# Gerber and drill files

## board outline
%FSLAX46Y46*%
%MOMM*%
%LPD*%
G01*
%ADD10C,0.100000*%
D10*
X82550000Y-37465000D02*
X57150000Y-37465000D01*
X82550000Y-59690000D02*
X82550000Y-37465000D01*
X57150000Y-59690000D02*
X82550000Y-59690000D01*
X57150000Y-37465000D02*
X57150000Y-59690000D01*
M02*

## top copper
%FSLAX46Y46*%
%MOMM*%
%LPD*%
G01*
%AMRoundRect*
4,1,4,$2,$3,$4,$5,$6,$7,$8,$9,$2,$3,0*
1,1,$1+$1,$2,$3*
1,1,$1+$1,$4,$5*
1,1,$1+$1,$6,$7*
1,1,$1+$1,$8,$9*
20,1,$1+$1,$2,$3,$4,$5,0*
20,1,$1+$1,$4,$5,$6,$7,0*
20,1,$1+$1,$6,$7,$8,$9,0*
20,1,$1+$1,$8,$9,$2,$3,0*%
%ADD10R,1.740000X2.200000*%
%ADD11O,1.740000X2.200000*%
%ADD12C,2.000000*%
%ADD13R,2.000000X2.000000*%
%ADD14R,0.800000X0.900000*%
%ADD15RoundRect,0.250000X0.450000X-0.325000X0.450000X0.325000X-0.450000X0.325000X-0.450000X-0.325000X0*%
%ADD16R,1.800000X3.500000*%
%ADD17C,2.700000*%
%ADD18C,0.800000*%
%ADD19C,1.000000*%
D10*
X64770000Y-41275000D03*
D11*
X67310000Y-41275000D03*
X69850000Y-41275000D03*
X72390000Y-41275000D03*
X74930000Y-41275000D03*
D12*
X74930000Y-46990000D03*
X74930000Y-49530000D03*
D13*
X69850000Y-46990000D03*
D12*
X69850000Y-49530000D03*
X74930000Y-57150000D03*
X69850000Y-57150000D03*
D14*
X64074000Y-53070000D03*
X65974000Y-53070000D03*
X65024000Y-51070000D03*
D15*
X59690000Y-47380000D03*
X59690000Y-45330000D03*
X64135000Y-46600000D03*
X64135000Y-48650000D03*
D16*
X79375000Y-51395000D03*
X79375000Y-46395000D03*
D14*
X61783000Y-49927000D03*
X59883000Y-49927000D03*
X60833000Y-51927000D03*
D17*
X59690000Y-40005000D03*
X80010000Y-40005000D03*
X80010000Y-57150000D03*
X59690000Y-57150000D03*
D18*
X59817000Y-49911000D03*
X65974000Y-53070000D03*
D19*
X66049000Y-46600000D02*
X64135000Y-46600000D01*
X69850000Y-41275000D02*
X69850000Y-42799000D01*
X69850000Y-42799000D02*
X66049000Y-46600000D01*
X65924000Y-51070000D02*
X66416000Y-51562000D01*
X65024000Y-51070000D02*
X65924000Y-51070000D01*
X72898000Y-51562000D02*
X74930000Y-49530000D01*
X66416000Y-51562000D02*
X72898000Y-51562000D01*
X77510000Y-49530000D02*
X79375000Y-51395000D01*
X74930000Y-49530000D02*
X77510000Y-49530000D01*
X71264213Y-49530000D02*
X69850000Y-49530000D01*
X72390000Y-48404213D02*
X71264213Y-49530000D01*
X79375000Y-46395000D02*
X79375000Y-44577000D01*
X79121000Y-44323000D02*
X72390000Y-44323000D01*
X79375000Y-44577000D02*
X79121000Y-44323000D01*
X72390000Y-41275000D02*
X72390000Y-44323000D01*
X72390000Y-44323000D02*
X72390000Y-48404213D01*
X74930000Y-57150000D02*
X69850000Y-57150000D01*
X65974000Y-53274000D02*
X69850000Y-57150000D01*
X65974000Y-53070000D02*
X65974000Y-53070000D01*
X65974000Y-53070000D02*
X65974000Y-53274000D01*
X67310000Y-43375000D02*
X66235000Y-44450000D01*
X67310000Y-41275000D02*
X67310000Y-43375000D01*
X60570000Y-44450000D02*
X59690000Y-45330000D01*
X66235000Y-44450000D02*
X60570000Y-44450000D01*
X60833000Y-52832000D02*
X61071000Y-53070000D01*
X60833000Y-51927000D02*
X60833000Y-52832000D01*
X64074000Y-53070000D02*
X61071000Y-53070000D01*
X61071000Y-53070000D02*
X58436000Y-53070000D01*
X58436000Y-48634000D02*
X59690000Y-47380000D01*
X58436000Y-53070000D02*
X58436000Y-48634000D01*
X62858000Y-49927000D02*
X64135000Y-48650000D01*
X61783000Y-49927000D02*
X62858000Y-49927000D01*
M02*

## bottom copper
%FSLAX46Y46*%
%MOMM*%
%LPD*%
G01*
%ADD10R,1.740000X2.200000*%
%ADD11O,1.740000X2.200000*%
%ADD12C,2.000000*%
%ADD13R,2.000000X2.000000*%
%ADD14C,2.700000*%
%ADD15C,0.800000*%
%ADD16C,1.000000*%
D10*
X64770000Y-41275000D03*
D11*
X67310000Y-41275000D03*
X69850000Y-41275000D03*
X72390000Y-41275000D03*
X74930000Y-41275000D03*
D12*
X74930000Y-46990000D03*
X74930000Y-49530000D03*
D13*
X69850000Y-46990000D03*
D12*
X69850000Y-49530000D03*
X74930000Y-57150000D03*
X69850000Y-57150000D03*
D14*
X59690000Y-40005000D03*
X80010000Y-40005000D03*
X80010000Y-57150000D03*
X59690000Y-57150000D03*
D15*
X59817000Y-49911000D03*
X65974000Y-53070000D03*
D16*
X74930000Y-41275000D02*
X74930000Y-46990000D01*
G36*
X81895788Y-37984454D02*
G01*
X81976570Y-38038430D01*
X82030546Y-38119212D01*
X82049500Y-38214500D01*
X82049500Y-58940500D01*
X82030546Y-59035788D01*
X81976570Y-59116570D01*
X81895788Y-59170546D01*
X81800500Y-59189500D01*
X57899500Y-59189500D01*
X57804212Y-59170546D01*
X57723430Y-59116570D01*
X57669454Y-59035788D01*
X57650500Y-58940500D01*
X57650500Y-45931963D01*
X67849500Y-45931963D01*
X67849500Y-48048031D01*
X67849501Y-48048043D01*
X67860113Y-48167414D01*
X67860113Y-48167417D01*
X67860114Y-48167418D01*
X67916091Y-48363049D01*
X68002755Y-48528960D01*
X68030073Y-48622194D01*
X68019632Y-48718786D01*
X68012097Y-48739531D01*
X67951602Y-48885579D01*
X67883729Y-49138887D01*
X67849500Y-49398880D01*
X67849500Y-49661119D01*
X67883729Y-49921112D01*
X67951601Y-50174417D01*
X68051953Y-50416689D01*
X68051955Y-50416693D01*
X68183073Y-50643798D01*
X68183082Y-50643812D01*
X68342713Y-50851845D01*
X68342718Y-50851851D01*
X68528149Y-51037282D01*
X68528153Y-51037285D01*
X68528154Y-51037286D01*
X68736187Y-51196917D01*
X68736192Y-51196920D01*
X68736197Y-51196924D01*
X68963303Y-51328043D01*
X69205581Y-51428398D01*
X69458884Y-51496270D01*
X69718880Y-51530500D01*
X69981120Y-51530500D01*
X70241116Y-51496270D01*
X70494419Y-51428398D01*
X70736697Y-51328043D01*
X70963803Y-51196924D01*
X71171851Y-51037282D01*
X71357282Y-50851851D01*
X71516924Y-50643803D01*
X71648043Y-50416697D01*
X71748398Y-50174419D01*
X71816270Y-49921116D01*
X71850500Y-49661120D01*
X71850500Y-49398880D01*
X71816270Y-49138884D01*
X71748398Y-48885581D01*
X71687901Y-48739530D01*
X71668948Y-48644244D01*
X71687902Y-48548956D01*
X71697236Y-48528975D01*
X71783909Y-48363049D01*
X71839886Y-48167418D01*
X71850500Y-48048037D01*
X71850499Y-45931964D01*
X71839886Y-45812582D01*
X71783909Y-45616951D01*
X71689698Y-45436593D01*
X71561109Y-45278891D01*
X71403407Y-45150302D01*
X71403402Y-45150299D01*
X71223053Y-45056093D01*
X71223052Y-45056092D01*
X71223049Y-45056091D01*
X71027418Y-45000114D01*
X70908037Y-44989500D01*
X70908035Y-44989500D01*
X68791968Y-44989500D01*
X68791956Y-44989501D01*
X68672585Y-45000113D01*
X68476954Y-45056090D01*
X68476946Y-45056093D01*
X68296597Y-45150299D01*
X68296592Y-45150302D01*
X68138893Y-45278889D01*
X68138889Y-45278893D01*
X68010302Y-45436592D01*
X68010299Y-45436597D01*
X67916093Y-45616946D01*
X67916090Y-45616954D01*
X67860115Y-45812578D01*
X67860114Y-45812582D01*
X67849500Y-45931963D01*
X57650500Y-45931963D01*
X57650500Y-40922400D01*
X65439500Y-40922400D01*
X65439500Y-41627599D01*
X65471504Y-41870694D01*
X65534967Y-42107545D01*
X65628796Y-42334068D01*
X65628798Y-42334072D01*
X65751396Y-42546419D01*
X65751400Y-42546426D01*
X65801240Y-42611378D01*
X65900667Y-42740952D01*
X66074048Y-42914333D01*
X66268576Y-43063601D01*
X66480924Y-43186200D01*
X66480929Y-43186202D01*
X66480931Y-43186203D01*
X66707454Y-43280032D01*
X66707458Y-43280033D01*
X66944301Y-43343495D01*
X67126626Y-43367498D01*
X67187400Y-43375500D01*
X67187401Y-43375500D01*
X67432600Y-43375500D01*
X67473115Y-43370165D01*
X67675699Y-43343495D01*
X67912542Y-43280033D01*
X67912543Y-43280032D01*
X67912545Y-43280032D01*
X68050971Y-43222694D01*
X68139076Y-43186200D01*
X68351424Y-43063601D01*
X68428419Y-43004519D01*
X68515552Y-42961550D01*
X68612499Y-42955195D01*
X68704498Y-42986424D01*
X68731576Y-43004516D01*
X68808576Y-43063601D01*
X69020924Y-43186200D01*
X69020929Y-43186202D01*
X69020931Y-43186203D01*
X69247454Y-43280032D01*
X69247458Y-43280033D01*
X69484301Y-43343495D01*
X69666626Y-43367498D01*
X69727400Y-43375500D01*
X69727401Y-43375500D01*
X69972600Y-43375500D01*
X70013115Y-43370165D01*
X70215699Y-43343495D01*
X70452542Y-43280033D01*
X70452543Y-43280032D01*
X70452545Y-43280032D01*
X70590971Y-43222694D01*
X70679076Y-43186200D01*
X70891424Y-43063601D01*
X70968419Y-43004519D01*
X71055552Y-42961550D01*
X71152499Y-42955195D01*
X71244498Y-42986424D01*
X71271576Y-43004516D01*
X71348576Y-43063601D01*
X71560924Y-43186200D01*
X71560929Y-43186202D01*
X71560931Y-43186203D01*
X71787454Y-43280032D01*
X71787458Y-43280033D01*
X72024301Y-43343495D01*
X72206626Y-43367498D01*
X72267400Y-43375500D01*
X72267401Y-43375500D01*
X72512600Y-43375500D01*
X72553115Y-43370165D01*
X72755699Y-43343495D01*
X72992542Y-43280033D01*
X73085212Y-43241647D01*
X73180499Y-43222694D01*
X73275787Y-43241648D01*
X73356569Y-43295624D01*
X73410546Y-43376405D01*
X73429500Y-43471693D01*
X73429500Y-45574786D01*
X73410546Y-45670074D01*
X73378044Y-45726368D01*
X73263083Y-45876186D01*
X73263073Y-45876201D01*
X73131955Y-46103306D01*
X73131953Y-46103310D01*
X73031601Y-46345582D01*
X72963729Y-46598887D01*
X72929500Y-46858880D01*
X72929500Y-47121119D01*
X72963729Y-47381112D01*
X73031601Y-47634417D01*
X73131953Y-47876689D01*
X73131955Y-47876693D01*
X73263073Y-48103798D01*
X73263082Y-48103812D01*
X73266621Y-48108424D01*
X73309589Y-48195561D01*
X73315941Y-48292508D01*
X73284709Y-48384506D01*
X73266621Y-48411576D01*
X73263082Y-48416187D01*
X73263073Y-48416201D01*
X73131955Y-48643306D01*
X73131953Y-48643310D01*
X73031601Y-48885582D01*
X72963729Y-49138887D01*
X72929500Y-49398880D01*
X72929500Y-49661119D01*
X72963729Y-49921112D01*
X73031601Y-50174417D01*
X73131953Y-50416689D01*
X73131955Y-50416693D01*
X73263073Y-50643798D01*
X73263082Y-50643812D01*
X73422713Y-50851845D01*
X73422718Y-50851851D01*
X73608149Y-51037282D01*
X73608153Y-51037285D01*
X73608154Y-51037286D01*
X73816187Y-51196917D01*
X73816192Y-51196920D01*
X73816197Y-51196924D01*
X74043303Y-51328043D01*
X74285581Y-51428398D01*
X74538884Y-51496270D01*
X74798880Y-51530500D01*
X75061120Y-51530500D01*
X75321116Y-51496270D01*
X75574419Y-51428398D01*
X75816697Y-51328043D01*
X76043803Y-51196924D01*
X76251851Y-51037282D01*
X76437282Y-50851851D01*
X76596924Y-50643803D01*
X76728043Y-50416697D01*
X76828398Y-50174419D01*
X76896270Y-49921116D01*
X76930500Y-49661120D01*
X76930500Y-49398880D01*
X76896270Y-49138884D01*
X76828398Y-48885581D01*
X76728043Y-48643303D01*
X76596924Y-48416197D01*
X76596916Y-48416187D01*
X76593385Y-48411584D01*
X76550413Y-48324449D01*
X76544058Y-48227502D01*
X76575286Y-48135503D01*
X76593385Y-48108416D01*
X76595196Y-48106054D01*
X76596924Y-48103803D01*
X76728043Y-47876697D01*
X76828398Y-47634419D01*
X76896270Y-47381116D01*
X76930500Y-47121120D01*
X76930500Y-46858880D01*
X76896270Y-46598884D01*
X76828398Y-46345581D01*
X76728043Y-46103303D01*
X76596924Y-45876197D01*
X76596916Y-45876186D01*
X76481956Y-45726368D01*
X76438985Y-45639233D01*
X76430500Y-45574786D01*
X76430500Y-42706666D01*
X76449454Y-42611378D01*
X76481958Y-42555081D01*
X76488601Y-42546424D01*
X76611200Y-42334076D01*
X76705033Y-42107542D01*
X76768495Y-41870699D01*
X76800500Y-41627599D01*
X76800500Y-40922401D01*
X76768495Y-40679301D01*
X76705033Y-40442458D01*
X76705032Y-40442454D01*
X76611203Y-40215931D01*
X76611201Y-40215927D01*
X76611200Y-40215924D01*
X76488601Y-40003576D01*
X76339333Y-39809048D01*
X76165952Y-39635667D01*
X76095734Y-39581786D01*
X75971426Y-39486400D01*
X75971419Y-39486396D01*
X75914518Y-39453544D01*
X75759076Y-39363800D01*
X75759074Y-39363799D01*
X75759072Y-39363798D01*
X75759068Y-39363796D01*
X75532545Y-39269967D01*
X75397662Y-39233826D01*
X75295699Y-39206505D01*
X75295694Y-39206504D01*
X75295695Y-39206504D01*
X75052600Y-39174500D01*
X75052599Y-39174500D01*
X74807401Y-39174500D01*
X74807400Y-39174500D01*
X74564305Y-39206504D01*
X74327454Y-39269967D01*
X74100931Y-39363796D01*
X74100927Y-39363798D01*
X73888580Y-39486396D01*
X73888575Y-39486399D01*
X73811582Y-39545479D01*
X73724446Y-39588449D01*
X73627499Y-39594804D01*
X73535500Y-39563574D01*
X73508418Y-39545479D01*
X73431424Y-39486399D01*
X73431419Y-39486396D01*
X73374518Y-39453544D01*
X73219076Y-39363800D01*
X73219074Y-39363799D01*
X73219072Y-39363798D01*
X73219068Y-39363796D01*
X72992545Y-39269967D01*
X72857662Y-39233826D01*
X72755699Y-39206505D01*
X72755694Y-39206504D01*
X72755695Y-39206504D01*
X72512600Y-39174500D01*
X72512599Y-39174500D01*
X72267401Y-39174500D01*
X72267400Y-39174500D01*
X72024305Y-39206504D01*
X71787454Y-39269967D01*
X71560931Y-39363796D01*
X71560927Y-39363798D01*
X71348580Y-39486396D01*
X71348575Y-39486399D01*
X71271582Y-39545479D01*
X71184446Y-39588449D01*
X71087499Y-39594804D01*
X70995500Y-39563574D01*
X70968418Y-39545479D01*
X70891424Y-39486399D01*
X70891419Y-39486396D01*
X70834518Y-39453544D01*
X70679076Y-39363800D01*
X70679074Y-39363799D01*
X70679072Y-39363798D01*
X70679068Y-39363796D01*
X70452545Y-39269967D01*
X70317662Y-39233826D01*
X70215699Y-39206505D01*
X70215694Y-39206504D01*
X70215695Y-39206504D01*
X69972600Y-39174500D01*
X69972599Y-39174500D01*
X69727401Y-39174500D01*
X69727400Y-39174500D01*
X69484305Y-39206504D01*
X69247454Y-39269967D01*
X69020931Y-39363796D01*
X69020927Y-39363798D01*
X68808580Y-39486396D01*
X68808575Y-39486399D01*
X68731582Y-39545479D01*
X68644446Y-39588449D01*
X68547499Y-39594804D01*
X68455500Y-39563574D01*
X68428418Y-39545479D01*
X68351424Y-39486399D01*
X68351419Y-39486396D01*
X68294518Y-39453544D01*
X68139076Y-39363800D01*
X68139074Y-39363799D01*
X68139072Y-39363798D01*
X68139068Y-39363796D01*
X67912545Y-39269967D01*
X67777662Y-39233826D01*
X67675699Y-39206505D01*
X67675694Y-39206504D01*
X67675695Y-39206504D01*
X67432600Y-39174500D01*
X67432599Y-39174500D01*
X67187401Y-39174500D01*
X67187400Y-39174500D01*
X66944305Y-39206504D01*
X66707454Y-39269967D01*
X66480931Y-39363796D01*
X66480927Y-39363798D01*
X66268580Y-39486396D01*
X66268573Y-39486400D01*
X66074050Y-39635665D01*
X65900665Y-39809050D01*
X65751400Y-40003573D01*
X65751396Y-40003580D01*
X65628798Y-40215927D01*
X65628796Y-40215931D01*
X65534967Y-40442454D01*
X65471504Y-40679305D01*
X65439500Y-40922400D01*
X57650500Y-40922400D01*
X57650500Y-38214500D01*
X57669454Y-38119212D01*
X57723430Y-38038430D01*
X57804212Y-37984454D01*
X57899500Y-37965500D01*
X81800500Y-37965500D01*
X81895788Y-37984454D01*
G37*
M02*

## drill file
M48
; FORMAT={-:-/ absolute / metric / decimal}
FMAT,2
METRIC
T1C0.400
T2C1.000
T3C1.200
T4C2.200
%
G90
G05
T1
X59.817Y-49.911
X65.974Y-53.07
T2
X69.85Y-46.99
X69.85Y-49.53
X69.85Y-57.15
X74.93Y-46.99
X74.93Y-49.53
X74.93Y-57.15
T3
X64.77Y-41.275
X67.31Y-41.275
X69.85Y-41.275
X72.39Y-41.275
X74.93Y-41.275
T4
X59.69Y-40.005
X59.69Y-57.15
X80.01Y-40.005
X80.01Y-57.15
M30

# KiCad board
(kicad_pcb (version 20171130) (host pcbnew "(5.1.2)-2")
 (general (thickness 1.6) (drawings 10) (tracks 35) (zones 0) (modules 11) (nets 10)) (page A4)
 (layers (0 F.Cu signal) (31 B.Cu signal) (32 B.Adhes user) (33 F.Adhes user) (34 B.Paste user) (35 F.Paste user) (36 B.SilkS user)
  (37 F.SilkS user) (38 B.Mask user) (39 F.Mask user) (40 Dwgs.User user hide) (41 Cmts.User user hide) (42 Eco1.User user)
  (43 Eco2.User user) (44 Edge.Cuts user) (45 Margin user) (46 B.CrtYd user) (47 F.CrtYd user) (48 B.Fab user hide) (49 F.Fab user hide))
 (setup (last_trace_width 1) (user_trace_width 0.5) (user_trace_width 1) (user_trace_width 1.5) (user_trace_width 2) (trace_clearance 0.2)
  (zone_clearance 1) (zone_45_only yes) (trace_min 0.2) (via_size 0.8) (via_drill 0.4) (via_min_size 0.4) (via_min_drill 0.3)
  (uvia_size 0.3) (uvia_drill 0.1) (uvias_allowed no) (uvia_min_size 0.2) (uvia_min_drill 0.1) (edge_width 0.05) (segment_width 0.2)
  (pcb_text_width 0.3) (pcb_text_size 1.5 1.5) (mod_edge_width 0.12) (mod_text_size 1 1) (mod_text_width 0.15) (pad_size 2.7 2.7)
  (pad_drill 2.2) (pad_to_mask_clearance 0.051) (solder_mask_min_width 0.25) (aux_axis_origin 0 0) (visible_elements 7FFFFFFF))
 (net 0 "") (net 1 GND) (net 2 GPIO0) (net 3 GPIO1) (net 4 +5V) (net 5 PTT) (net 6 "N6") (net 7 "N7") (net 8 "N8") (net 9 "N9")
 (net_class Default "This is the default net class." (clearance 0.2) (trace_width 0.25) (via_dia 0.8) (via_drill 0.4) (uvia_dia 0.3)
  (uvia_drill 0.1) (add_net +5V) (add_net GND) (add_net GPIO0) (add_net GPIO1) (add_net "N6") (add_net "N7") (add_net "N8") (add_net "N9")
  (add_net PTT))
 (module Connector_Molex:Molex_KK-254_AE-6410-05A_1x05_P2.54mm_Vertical (layer F.Cu) (at 64.77 41.275)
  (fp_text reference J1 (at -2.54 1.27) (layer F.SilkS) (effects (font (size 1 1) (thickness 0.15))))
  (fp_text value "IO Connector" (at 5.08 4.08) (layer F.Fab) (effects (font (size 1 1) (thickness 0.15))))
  (pad 1 thru_hole rect (at 0 0) (size 1.74 2.2) (drill 1.2) (layers *.Cu *.Mask) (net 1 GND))
  (pad 2 thru_hole oval (at 2.54 0) (size 1.74 2.2) (drill 1.2) (layers *.Cu *.Mask) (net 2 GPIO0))
  (pad 3 thru_hole oval (at 5.08 0) (size 1.74 2.2) (drill 1.2) (layers *.Cu *.Mask) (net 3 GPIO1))
  (pad 4 thru_hole oval (at 7.62 0) (size 1.74 2.2) (drill 1.2) (layers *.Cu *.Mask) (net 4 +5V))
  (pad 5 thru_hole oval (at 10.16 0) (size 1.74 2.2) (drill 1.2) (layers *.Cu *.Mask) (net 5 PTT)))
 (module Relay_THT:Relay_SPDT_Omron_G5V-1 (layer F.Cu) (at 69.85 46.99)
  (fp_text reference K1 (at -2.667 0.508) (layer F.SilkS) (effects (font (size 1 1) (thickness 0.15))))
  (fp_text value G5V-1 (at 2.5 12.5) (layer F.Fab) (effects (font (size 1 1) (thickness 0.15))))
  (pad 10 thru_hole circle (at 5.08 0) (size 2 2) (drill 1) (layers *.Cu *.Mask) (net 5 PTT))
  (pad 9 thru_hole circle (at 5.08 2.54) (size 2 2) (drill 1) (layers *.Cu *.Mask) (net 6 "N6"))
  (pad 1 thru_hole rect (at 0 0) (size 2 2) (drill 1) (layers *.Cu *.Mask) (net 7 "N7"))
  (pad 2 thru_hole circle (at 0 2.54) (size 2 2) (drill 1) (layers *.Cu *.Mask) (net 4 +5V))
  (pad 6 thru_hole circle (at 5.08 10.16) (size 2 2) (drill 1) (layers *.Cu *.Mask) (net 1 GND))
  (pad 5 thru_hole circle (at 0 10.16) (size 2 2) (drill 1) (layers *.Cu *.Mask) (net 1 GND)))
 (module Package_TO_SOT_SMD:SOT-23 (layer F.Cu) (at 65.024 52.07 90)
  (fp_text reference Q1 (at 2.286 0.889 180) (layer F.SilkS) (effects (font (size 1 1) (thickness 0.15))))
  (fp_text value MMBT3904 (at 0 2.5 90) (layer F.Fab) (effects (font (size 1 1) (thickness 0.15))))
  (pad 1 smd rect (at -1 -0.95 90) (size 0.9 0.8) (layers F.Cu F.Paste F.Mask) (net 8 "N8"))
  (pad 2 smd rect (at -1 0.95 90) (size 0.9 0.8) (layers F.Cu F.Paste F.Mask) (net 1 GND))
  (pad 3 smd rect (at 1 0 90) (size 0.9 0.8) (layers F.Cu F.Paste F.Mask) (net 6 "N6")))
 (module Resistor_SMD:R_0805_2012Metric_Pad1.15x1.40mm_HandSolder (layer F.Cu) (at 59.69 46.355 90)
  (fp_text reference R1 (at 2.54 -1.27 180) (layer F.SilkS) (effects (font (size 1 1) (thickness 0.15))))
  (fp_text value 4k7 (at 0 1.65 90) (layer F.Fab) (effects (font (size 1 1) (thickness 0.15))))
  (pad 1 smd roundrect (at -1.025 0 90) (size 1.15 1.4) (layers F.Cu F.Paste F.Mask) (roundrect_rratio 0.217391) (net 8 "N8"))
  (pad 2 smd roundrect (at 1.025 0 90) (size 1.15 1.4) (layers F.Cu F.Paste F.Mask) (roundrect_rratio 0.217391) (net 2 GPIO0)))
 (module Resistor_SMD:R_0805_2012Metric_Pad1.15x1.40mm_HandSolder (layer F.Cu) (at 64.135 47.625 90)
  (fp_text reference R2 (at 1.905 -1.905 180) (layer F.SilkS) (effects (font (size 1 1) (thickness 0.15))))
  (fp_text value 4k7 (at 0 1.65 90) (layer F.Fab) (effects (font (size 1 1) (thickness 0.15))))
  (pad 2 smd roundrect (at 1.025 0 90) (size 1.15 1.4) (layers F.Cu F.Paste F.Mask) (roundrect_rratio 0.217391) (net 3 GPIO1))
  (pad 1 smd roundrect (at -1.025 0 90) (size 1.15 1.4) (layers F.Cu F.Paste F.Mask) (roundrect_rratio 0.217391) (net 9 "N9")))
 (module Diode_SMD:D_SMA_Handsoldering (layer F.Cu) (at 79.375 48.895 90)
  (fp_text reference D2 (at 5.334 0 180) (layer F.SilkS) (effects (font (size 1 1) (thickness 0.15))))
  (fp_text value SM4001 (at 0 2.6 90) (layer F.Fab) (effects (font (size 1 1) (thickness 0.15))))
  (pad 1 smd rect (at -2.5 0 90) (size 3.5 1.8) (layers F.Cu F.Paste F.Mask) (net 6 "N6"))
  (pad 2 smd rect (at 2.5 0 90) (size 3.5 1.8) (layers F.Cu F.Paste F.Mask) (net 4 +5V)))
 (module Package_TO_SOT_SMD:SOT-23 (layer F.Cu) (at 60.833 50.927 270)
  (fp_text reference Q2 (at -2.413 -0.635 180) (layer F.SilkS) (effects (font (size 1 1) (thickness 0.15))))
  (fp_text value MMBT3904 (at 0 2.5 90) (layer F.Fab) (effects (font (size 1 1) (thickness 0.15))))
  (pad 1 smd rect (at -1 -0.95 270) (size 0.9 0.8) (layers F.Cu F.Paste F.Mask) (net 9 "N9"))
  (pad 2 smd rect (at -1 0.95 270) (size 0.9 0.8) (layers F.Cu F.Paste F.Mask) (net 1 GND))
  (pad 3 smd rect (at 1 0 270) (size 0.9 0.8) (layers F.Cu F.Paste F.Mask) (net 8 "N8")))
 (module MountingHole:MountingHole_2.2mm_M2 (layer F.Cu) (at 59.69 40.005)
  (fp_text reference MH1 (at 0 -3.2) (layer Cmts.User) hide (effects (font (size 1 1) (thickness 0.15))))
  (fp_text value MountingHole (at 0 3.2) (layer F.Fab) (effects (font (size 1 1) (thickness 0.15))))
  (pad "" thru_hole circle (at 0 0) (size 2.7 2.7) (drill 2.2) (layers *.Cu *.Mask) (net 1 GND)))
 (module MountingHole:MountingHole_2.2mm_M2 (layer F.Cu) (at 80.01 40.005)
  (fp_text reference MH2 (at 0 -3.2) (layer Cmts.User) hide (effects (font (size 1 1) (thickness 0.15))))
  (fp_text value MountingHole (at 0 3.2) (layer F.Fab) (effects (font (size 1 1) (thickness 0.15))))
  (pad 1 thru_hole circle (at 0 0) (size 2.7 2.7) (drill 2.2) (layers *.Cu *.Mask) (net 1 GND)))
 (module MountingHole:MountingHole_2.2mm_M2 (layer F.Cu) (at 80.01 57.15)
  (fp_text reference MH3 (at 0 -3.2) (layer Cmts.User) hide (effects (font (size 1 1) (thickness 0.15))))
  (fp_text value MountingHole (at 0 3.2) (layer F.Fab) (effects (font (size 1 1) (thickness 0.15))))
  (pad "" thru_hole circle (at 0 0) (size 2.7 2.7) (drill 2.2) (layers *.Cu *.Mask) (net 1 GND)))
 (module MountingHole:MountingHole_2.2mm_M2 (layer F.Cu) (at 59.69 57.15)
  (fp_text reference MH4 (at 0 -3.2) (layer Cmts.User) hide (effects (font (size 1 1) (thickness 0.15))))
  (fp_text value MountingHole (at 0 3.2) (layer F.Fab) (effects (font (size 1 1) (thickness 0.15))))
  (pad "" thru_hole circle (at 0 0) (size 2.7 2.7) (drill 2.2) (layers *.Cu *.Mask) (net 1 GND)))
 (gr_line (start 82.55 37.465) (end 57.15 37.465) (layer Edge.Cuts) (width 0.1))
 (gr_line (start 82.55 59.69) (end 82.55 37.465) (layer Edge.Cuts) (width 0.1))
 (gr_line (start 57.15 59.69) (end 82.55 59.69) (layer Edge.Cuts) (width 0.1))
 (gr_line (start 57.15 37.465) (end 57.15 59.69) (layer Edge.Cuts) (width 0.1))
 (via (at 59.817 49.911) (size 0.8) (drill 0.4) (layers F.Cu B.Cu) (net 1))
 (segment (start 66.049 46.6) (end 64.135 46.6) (width 1) (layer F.Cu) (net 3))
 (segment (start 69.85 41.275) (end 69.85 42.799) (width 1) (layer F.Cu) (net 3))
 (segment (start 69.85 42.799) (end 66.049 46.6) (width 1) (layer F.Cu) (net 3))
 (segment (start 65.924 51.07) (end 66.416 51.562) (width 1) (layer F.Cu) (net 6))
 (segment (start 65.024 51.07) (end 65.924 51.07) (width 1) (layer F.Cu) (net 6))
 (segment (start 72.898 51.562) (end 74.93 49.53) (width 1) (layer F.Cu) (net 6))
 (segment (start 66.416 51.562) (end 72.898 51.562) (width 1) (layer F.Cu) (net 6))
 (segment (start 77.51 49.53) (end 79.375 51.395) (width 1) (layer F.Cu) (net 6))
 (segment (start 74.93 49.53) (end 77.51 49.53) (width 1) (layer F.Cu) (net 6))
 (segment (start 71.264213 49.53) (end 69.85 49.53) (width 1) (layer F.Cu) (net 4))
 (segment (start 72.39 48.404213) (end 71.264213 49.53) (width 1) (layer F.Cu) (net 4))
 (segment (start 79.375 46.395) (end 79.375 44.577) (width 1) (layer F.Cu) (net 4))
 (segment (start 79.121 44.323) (end 72.39 44.323) (width 1) (layer F.Cu) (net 4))
 (segment (start 79.375 44.577) (end 79.121 44.323) (width 1) (layer F.Cu) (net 4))
 (segment (start 72.39 41.275) (end 72.39 44.323) (width 1) (layer F.Cu) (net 4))
 (segment (start 72.39 44.323) (end 72.39 48.404213) (width 1) (layer F.Cu) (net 4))
 (segment (start 74.93 57.15) (end 69.85 57.15) (width 1) (layer F.Cu) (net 1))
 (segment (start 65.974 53.274) (end 69.85 57.15) (width 1) (layer F.Cu) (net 1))
 (segment (start 65.974 53.07) (end 65.974 53.07) (width 1) (layer F.Cu) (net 1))
 (segment (start 65.974 53.07) (end 65.974 53.274) (width 1) (layer F.Cu) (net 1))
 (via (at 65.974 53.07) (size 0.8) (drill 0.4) (layers F.Cu B.Cu) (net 1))
 (segment (start 67.31 43.375) (end 66.235 44.45) (width 1) (layer F.Cu) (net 2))
 (segment (start 67.31 41.275) (end 67.31 43.375) (width 1) (layer F.Cu) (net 2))
 (segment (start 60.57 44.45) (end 59.69 45.33) (width 1) (layer F.Cu) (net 2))
 (segment (start 66.235 44.45) (end 60.57 44.45) (width 1) (layer F.Cu) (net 2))
 (segment (start 74.93 41.275) (end 74.93 46.99) (width 1) (layer B.Cu) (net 5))
 (segment (start 60.833 52.832) (end 61.071 53.07) (width 1) (layer F.Cu) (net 8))
 (segment (start 60.833 51.927) (end 60.833 52.832) (width 1) (layer F.Cu) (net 8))
 (segment (start 64.074 53.07) (end 61.071 53.07) (width 1) (layer F.Cu) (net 8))
 (segment (start 61.071 53.07) (end 58.436 53.07) (width 1) (layer F.Cu) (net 8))
 (segment (start 58.436 48.634) (end 59.69 47.38) (width 1) (layer F.Cu) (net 8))
 (segment (start 58.436 53.07) (end 58.436 48.634) (width 1) (layer F.Cu) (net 8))
 (segment (start 62.858 49.927) (end 64.135 48.65) (width 1) (layer F.Cu) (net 9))
 (segment (start 61.783 49.927) (end 62.858 49.927) (width 1) (layer F.Cu) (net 9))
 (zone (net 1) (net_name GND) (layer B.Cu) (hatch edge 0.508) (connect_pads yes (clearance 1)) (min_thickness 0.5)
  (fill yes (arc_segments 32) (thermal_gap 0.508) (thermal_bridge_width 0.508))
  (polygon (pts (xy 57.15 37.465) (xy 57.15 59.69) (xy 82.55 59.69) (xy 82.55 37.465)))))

